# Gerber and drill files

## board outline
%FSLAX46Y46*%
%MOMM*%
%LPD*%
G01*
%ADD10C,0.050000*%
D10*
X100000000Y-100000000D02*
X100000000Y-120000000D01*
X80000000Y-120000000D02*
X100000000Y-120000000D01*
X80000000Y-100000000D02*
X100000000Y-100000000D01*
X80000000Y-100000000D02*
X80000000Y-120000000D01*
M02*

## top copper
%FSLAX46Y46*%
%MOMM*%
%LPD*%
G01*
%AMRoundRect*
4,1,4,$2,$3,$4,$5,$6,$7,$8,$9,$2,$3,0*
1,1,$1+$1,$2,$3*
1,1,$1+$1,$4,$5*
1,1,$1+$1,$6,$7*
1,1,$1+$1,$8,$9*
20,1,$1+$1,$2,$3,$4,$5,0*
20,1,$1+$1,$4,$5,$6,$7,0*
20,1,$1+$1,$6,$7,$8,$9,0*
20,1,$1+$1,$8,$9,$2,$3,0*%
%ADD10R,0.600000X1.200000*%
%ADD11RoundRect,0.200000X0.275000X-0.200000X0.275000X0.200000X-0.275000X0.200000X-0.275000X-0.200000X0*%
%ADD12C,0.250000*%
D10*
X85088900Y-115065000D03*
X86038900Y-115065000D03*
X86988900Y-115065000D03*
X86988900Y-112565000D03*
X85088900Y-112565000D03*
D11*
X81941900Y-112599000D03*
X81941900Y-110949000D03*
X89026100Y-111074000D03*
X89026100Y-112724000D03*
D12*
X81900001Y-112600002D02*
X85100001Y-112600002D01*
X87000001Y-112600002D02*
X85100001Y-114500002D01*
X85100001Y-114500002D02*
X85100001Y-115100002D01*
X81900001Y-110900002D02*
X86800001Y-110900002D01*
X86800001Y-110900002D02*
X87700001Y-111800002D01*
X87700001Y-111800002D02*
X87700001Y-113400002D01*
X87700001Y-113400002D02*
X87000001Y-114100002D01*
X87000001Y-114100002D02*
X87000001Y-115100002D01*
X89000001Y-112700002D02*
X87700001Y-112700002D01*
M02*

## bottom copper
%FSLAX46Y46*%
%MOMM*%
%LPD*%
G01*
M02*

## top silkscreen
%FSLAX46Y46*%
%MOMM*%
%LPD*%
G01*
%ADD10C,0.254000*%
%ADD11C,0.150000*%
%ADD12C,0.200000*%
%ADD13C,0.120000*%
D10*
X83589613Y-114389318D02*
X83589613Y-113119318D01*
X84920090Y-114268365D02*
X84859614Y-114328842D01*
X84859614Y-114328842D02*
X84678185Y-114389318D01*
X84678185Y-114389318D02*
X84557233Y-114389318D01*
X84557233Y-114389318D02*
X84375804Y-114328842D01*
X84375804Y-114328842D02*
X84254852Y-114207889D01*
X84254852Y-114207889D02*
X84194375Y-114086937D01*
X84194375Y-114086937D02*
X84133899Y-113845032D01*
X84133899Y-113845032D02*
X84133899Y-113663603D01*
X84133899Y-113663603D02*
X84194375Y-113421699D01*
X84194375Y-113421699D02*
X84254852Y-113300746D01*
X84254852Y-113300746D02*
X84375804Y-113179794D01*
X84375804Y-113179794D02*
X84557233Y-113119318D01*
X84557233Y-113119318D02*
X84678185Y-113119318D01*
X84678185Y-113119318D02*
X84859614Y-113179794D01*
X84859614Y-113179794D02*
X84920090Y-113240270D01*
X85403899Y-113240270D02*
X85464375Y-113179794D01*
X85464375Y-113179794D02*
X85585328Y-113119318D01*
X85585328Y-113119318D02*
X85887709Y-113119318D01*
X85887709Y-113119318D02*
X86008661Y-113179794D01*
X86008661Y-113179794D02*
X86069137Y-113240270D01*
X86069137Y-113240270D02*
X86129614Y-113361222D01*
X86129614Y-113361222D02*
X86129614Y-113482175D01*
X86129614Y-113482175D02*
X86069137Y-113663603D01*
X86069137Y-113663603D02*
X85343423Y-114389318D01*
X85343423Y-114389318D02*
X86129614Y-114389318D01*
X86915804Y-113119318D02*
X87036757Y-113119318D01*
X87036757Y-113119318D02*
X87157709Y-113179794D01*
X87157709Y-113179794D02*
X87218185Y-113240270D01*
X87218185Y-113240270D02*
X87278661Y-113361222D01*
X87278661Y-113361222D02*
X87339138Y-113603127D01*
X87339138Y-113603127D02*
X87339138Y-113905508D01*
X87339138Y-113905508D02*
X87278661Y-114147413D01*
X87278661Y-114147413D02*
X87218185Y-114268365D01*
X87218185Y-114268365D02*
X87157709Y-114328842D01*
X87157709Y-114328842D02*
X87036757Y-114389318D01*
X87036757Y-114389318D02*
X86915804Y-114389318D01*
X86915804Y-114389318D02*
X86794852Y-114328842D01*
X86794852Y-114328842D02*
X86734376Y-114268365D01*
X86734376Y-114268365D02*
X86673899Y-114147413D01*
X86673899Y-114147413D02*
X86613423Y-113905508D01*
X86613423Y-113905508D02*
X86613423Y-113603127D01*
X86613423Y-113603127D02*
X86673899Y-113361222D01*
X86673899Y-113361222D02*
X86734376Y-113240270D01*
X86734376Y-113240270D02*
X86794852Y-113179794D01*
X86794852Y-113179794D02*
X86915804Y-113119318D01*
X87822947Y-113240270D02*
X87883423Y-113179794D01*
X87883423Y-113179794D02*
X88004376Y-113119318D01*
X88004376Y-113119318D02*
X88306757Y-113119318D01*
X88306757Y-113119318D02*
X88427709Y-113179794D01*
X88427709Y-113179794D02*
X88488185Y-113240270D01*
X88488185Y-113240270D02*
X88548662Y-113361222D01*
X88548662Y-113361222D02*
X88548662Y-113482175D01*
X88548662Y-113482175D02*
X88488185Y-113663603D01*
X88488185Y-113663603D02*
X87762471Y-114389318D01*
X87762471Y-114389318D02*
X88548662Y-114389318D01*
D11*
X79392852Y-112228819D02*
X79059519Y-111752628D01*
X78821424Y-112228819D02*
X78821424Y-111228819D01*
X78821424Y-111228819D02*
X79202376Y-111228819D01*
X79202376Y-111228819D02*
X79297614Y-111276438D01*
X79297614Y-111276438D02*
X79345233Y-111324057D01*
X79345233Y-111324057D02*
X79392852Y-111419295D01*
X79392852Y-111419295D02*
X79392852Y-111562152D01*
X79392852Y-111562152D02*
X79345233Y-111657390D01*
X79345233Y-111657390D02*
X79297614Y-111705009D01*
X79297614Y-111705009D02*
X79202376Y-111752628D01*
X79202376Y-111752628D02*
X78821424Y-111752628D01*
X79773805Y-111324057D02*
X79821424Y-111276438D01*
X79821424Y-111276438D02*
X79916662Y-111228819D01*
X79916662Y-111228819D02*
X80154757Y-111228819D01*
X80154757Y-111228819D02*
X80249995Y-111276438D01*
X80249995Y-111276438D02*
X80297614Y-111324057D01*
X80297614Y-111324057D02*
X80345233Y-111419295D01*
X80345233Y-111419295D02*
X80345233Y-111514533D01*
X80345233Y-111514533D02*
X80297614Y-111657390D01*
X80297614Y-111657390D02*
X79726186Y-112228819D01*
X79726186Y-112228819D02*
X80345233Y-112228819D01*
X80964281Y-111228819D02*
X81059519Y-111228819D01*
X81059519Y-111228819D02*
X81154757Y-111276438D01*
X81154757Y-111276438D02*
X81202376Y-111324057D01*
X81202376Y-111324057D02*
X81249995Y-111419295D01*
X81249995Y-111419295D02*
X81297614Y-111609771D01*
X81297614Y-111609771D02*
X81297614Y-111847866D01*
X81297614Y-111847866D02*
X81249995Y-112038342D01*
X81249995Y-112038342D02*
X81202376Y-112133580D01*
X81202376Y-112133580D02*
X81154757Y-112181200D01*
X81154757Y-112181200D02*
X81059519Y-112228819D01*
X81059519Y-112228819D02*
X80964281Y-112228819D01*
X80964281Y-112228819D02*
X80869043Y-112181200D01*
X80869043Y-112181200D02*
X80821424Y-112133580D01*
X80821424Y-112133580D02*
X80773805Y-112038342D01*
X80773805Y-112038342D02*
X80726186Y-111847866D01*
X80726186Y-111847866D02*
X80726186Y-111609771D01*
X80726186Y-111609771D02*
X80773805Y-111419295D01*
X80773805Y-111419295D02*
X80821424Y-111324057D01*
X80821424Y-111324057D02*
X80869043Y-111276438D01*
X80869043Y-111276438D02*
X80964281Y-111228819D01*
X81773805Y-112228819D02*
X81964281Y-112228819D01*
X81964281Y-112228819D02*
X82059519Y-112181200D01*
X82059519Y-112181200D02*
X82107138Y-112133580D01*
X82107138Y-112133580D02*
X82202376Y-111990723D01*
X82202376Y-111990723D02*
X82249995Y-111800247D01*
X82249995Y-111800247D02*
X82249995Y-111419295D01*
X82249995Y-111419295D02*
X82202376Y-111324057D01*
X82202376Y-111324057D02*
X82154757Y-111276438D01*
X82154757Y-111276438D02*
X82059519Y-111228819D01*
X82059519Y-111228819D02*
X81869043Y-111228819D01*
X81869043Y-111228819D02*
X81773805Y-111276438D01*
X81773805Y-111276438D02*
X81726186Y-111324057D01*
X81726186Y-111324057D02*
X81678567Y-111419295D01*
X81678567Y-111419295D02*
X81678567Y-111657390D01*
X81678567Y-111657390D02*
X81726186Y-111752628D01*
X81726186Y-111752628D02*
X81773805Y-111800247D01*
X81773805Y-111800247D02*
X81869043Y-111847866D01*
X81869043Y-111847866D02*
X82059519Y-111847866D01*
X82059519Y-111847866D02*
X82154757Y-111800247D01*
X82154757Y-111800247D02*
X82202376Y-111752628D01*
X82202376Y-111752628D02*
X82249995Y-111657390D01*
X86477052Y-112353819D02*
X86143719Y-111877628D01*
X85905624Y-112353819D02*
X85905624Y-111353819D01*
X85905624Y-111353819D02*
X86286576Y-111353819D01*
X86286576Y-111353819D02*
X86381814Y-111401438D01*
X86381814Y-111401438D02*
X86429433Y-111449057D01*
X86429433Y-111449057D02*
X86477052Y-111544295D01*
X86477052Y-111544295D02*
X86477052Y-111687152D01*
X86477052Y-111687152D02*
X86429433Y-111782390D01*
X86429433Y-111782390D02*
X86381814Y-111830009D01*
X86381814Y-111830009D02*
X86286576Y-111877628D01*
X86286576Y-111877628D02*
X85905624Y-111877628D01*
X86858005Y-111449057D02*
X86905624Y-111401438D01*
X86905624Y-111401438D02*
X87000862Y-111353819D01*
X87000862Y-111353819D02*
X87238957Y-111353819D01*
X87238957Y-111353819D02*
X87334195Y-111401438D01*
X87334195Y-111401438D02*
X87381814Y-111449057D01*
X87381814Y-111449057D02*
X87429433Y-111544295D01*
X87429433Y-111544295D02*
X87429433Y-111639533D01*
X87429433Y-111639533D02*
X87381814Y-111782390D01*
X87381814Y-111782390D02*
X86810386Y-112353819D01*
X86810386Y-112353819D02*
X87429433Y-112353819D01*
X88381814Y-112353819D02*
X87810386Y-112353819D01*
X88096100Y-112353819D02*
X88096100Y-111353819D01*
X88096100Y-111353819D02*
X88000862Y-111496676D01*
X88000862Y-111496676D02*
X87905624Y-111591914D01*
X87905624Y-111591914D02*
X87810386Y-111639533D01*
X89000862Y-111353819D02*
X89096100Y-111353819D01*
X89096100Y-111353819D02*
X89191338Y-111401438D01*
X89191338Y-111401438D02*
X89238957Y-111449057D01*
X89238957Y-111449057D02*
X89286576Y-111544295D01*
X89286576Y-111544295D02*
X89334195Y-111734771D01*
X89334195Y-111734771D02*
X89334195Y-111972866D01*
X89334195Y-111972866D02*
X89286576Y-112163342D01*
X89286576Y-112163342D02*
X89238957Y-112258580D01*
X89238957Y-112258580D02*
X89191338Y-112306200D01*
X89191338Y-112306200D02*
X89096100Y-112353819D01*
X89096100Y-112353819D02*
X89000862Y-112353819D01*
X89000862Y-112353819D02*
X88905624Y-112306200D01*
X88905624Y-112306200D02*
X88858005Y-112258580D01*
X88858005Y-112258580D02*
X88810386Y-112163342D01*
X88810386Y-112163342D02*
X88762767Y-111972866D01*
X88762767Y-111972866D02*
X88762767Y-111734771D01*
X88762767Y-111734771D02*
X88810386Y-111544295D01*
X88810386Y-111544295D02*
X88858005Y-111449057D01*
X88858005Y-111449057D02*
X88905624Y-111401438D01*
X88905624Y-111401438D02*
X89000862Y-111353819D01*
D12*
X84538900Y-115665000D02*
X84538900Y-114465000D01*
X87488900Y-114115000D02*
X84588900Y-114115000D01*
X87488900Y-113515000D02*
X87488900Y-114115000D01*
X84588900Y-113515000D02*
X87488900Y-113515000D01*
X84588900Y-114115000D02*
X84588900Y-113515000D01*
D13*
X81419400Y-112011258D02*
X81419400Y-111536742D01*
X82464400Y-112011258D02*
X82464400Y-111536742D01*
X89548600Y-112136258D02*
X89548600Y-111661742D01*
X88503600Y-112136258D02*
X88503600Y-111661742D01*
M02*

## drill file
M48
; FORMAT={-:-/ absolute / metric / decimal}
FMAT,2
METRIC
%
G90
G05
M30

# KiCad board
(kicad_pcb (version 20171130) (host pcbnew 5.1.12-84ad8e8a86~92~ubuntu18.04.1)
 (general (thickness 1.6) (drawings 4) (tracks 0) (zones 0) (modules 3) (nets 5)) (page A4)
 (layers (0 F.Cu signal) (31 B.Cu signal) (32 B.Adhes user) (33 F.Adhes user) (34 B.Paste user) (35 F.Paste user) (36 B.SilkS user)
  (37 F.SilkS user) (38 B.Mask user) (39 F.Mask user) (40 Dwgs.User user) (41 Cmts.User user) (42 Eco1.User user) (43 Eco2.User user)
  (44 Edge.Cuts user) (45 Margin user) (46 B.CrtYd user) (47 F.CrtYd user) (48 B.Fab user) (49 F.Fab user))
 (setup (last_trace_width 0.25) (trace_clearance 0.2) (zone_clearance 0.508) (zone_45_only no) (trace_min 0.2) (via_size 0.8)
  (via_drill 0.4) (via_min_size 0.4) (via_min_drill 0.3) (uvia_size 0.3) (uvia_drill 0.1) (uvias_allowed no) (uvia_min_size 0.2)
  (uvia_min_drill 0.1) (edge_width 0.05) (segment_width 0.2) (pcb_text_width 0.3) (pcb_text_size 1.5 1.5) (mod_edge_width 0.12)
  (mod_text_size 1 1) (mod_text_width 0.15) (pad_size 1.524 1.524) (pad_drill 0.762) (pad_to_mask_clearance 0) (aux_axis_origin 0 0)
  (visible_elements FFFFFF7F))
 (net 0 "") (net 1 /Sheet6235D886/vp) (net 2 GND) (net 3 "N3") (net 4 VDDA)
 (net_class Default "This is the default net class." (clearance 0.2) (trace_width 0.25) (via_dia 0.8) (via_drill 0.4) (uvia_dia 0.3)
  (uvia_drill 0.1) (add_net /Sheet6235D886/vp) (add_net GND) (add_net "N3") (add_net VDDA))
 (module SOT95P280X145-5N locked (layer F.Cu) (at 86.038900 113.815000 90.000000)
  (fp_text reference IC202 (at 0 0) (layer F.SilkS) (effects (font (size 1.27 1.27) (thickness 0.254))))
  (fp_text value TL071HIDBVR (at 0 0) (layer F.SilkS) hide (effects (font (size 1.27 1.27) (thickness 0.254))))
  (fp_line (start -1.85 -1.5) (end -0.65 -1.5) (layer F.SilkS) (width 0.2))
  (fp_line (start -0.3 1.45) (end -0.3 -1.45) (layer F.SilkS) (width 0.2))
  (fp_line (start 0.3 1.45) (end -0.3 1.45) (layer F.SilkS) (width 0.2))
  (fp_line (start 0.3 -1.45) (end 0.3 1.45) (layer F.SilkS) (width 0.2))
  (fp_line (start -0.3 -1.45) (end 0.3 -1.45) (layer F.SilkS) (width 0.2))
  (pad 1 smd rect (at -1.25 -0.95 180.000000) (size 0.6 1.2) (layers F.Cu F.Mask F.Paste) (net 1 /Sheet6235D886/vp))
  (pad 2 smd rect (at -1.25 0 180.000000) (size 0.6 1.2) (layers F.Cu F.Mask F.Paste) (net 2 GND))
  (pad 3 smd rect (at -1.25 0.95 180.000000) (size 0.6 1.2) (layers F.Cu F.Mask F.Paste) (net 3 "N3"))
  (pad 4 smd rect (at 1.25 0.95 180.000000) (size 0.6 1.2) (layers F.Cu F.Mask F.Paste) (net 1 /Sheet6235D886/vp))
  (pad 5 smd rect (at 1.25 -0.95 180.000000) (size 0.6 1.2) (layers F.Cu F.Mask F.Paste) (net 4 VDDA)))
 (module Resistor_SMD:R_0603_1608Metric (layer F.Cu) (at 81.941900 111.774000 90.000000)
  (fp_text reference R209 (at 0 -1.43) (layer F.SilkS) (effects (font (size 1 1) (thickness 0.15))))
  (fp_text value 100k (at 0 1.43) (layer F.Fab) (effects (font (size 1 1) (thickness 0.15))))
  (fp_line (start -0.237258 -0.5225) (end 0.237258 -0.5225) (layer F.SilkS) (width 0.12))
  (fp_line (start -0.237258 0.5225) (end 0.237258 0.5225) (layer F.SilkS) (width 0.12))
  (pad 1 smd roundrect (at -0.825 0 90.000000) (size 0.8 0.95) (layers F.Cu F.Mask F.Paste) (roundrect_rratio 0.25) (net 4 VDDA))
  (pad 2 smd roundrect (at 0.825 0 90.000000) (size 0.8 0.95) (layers F.Cu F.Mask F.Paste) (roundrect_rratio 0.25) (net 3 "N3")))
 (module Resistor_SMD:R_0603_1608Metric (layer F.Cu) (at 89.026100 111.899000 90.000000)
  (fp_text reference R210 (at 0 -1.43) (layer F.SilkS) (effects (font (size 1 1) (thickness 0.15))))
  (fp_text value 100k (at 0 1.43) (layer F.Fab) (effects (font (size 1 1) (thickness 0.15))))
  (fp_line (start -0.237258 0.5225) (end 0.237258 0.5225) (layer F.SilkS) (width 0.12))
  (fp_line (start -0.237258 -0.5225) (end 0.237258 -0.5225) (layer F.SilkS) (width 0.12))
  (pad 2 smd roundrect (at 0.825 0 90.000000) (size 0.8 0.95) (layers F.Cu F.Mask F.Paste) (roundrect_rratio 0.25) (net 2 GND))
  (pad 1 smd roundrect (at -0.825 0 90.000000) (size 0.8 0.95) (layers F.Cu F.Mask F.Paste) (roundrect_rratio 0.25) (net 3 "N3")))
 (gr_line (start 100 100) (end 100 120) (layer Edge.Cuts) (width 0.05))
 (gr_line (start 80 120) (end 100 120) (layer Edge.Cuts) (width 0.05))
 (gr_line (start 80 100) (end 100 100) (layer Edge.Cuts) (width 0.05))
 (gr_line (start 80 100) (end 80 120) (layer Edge.Cuts) (width 0.05))
 (segment (start 81.900001 112.600002) (end 85.100001 112.600002) (width 0.250000) (layer F.Cu) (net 4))
 (segment (start 87.000001 112.600002) (end 85.100001 114.500002) (width 0.250000) (layer F.Cu) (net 1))
 (segment (start 85.100001 114.500002) (end 85.100001 115.100002) (width 0.250000) (layer F.Cu) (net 1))
 (segment (start 81.900001 110.900002) (end 86.800001 110.900002) (width 0.250000) (layer F.Cu) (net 3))
 (segment (start 86.800001 110.900002) (end 87.700001 111.800002) (width 0.250000) (layer F.Cu) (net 3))
 (segment (start 87.700001 111.800002) (end 87.700001 113.400002) (width 0.250000) (layer F.Cu) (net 3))
 (segment (start 87.700001 113.400002) (end 87.000001 114.100002) (width 0.250000) (layer F.Cu) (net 3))
 (segment (start 87.000001 114.100002) (end 87.000001 115.100002) (width 0.250000) (layer F.Cu) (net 3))
 (segment (start 89.000001 112.700002) (end 87.700001 112.700002) (width 0.250000) (layer F.Cu) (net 3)))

